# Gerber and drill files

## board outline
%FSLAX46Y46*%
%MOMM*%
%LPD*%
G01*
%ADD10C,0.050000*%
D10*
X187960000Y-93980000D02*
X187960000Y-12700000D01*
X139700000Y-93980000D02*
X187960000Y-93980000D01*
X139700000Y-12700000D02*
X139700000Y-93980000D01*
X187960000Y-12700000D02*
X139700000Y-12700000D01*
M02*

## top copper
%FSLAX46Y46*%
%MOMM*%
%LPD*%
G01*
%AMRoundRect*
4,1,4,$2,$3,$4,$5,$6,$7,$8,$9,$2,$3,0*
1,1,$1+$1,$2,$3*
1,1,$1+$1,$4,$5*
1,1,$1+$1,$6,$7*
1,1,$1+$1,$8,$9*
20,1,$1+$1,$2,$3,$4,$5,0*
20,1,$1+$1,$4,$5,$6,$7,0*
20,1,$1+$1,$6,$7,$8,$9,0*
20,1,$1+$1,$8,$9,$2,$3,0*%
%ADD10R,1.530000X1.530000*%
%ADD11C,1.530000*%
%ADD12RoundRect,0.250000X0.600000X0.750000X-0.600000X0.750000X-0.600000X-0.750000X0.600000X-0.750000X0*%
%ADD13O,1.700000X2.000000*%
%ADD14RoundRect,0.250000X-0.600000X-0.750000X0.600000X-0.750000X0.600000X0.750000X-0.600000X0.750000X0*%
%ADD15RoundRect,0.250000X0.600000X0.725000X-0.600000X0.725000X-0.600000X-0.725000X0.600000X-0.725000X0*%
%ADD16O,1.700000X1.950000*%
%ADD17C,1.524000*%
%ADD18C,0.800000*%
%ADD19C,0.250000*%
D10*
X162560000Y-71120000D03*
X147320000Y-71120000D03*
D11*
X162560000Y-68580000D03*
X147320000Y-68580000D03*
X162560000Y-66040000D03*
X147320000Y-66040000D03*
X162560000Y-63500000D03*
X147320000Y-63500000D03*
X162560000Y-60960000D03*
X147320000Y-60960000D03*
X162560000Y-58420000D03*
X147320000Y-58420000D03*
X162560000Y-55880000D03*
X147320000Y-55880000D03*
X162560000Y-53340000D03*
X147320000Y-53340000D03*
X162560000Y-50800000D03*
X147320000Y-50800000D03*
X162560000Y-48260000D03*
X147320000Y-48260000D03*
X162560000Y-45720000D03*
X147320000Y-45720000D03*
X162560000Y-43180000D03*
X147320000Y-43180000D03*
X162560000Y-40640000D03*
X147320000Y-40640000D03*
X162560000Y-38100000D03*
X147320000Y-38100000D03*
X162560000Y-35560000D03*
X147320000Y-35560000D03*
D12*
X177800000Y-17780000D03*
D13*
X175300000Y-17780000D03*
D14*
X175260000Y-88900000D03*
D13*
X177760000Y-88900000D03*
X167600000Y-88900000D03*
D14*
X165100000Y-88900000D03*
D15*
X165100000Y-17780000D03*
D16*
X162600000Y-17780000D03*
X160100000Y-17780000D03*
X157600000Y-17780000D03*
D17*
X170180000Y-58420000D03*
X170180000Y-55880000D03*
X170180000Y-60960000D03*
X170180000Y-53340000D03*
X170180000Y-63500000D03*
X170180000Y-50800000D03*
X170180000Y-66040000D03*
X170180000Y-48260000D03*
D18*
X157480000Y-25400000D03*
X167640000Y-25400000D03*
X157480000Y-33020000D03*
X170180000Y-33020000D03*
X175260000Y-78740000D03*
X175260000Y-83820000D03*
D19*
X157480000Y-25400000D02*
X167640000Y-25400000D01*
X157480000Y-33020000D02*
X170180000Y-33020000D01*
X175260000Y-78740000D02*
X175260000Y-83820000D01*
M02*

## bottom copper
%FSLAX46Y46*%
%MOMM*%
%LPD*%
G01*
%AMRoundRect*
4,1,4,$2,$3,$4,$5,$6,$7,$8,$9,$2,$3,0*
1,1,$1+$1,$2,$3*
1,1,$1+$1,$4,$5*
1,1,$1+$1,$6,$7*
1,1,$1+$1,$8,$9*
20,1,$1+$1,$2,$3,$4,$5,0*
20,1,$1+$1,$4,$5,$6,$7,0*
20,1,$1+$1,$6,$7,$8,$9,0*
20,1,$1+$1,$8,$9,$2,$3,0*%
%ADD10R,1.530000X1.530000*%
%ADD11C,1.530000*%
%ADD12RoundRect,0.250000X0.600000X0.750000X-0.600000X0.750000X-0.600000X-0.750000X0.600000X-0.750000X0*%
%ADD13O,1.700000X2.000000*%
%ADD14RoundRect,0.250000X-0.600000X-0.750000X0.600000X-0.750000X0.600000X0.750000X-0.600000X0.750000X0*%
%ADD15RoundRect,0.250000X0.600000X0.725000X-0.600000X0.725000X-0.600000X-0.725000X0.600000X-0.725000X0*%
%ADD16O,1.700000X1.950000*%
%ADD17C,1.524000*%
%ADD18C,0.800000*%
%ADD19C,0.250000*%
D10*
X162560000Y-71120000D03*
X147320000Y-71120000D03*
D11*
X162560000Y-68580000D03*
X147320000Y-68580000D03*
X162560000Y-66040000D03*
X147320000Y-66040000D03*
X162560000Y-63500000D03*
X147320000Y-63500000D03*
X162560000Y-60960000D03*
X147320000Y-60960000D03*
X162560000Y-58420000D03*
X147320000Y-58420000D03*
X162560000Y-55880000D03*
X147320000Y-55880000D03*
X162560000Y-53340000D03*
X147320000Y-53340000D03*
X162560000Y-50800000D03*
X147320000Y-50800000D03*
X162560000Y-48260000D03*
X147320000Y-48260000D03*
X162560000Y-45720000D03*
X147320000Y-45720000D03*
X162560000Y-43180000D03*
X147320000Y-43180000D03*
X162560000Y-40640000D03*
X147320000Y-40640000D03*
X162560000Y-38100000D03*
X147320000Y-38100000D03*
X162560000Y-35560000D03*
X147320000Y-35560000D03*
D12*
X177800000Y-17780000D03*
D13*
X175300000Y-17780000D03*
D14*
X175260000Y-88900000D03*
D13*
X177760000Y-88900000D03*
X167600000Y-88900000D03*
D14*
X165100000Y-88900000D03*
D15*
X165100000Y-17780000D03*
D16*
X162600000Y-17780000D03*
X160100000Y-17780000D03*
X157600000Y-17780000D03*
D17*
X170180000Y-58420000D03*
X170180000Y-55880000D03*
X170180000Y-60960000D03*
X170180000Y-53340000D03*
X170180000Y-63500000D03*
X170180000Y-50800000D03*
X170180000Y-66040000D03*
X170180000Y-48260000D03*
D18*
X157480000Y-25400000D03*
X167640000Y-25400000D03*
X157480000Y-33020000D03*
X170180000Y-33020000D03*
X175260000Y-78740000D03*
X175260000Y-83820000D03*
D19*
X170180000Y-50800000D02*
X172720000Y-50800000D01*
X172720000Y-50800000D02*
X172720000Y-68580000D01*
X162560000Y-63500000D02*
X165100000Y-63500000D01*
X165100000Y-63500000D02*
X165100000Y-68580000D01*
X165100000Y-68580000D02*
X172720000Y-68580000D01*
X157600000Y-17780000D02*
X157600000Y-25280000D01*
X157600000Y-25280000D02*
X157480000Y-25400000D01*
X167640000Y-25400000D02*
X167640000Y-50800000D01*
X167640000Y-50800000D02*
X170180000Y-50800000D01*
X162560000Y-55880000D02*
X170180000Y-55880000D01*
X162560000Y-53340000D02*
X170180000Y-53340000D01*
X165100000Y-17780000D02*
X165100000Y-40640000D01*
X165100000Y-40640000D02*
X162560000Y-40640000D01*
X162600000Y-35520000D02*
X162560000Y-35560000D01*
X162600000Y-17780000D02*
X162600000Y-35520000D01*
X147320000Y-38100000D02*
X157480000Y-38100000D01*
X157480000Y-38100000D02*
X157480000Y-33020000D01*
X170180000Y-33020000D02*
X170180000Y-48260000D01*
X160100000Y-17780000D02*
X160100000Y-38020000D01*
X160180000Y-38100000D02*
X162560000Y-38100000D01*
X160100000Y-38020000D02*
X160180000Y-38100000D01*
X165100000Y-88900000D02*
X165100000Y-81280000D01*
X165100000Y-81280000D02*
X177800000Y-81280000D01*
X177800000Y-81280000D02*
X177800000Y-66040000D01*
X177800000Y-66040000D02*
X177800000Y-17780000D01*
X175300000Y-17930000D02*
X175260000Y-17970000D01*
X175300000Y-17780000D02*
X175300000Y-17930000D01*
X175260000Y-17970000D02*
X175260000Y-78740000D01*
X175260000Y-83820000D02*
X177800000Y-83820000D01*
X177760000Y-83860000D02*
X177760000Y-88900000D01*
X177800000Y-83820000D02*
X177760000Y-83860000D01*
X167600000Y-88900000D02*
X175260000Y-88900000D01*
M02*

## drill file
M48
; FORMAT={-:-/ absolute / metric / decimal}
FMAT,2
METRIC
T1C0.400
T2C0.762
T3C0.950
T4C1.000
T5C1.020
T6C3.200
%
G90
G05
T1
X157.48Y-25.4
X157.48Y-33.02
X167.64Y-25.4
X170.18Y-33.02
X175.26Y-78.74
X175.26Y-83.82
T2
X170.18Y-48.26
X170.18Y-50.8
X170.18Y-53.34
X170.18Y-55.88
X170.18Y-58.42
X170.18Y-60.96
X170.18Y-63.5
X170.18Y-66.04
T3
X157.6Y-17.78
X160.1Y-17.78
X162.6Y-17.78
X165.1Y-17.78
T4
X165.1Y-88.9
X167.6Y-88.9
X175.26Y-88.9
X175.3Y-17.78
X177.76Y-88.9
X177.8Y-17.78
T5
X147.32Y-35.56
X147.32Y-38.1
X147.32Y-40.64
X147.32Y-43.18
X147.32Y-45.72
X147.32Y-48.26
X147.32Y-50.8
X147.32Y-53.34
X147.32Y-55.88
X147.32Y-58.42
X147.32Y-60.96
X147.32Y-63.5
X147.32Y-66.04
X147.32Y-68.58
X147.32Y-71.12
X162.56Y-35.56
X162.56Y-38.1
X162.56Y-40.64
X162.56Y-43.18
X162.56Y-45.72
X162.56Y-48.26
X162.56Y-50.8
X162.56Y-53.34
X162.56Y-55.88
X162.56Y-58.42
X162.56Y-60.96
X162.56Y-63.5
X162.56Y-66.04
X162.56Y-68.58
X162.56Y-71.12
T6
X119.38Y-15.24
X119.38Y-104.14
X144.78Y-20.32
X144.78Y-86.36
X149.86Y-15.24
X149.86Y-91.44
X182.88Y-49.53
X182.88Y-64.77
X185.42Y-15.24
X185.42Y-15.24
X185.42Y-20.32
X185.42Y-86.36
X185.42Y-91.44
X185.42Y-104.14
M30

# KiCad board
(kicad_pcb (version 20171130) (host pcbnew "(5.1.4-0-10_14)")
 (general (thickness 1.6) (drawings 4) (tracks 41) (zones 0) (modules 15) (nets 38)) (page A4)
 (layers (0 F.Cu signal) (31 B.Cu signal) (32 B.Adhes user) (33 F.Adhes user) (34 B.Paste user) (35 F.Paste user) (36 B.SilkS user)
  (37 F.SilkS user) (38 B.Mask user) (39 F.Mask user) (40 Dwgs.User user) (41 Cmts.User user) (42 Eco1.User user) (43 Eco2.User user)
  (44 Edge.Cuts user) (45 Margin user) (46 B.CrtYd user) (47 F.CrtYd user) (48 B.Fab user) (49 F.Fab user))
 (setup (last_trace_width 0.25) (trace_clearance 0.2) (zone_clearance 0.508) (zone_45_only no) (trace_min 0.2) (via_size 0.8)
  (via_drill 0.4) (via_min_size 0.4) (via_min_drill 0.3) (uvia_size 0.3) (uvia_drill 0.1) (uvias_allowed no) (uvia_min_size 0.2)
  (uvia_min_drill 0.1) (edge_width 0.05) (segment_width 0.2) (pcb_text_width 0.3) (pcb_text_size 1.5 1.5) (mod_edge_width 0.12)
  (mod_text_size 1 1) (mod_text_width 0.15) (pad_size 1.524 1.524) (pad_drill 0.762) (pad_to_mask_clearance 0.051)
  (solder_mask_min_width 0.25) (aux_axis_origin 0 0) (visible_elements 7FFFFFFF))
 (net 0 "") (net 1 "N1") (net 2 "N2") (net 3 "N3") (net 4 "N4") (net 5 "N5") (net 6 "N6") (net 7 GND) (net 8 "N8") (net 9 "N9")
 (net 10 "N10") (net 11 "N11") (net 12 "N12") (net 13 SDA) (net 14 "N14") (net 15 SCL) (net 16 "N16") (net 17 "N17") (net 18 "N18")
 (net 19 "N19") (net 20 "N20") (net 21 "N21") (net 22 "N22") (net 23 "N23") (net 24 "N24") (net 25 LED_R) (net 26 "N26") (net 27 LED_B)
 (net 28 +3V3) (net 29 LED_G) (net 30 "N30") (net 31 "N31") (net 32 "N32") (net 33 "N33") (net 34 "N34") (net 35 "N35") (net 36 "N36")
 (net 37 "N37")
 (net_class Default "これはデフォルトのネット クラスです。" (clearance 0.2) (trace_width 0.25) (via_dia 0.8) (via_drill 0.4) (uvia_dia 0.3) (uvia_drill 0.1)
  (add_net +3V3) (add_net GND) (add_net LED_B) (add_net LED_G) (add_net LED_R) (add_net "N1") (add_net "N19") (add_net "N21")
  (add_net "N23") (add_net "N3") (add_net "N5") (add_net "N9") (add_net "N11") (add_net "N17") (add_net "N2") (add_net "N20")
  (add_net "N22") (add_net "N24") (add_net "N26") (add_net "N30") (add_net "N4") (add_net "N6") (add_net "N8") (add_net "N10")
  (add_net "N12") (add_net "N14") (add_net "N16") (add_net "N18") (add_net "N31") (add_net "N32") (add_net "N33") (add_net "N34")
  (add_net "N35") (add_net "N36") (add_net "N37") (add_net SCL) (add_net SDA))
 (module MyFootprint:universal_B (layer F.Cu) (at 152.4 58.42 90)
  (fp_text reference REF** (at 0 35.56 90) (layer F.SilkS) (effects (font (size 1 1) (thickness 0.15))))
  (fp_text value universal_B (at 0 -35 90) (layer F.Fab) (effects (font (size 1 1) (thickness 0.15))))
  (pad "" np_thru_hole circle (at 43.18 -33.02 90) (size 3.2 3.2) (drill 3.2) (layers *.Cu *.Mask))
  (pad "" np_thru_hole circle (at 43.18 33.02 90) (size 3.2 3.2) (drill 3.2) (layers *.Cu *.Mask))
  (pad "" np_thru_hole circle (at -45.72 33.02 90) (size 3.2 3.2) (drill 3.2) (layers *.Cu *.Mask))
  (pad "" np_thru_hole circle (at -45.72 -33.02 90) (size 3.2 3.2) (drill 3.2) (layers *.Cu *.Mask)))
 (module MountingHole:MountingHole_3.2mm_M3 (layer F.Cu) (at 144.78 86.36)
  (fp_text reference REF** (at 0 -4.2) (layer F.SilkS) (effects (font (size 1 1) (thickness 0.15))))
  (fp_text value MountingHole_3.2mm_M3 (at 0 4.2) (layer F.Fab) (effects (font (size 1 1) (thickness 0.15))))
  (pad 1 np_thru_hole circle (at 0 0) (size 3.2 3.2) (drill 3.2) (layers *.Cu *.Mask)))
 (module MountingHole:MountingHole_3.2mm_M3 (layer F.Cu) (at 185.42 86.36)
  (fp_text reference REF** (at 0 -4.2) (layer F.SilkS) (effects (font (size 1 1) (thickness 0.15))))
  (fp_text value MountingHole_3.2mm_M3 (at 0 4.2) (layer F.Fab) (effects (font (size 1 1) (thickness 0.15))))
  (pad 1 np_thru_hole circle (at 0 0) (size 3.2 3.2) (drill 3.2) (layers *.Cu *.Mask)))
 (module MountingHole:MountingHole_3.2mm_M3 (layer F.Cu) (at 144.78 20.32)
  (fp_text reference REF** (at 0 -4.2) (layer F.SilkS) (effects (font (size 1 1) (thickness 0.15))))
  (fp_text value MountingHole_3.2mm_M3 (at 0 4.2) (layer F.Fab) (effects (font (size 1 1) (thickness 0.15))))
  (pad 1 np_thru_hole circle (at 0 0) (size 3.2 3.2) (drill 3.2) (layers *.Cu *.Mask)))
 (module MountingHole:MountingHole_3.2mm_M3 (layer F.Cu) (at 185.42 20.32)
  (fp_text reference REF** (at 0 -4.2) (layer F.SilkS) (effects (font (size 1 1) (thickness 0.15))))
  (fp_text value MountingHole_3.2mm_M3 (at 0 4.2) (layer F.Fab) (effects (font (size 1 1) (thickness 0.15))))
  (pad 1 np_thru_hole circle (at 0 0) (size 3.2 3.2) (drill 3.2) (layers *.Cu *.Mask)))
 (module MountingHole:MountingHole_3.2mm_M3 (layer F.Cu) (at 149.86 91.44)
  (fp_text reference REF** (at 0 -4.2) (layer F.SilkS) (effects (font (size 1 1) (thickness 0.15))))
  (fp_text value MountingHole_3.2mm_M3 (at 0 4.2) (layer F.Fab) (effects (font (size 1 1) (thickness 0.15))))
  (pad 1 np_thru_hole circle (at 0 0) (size 3.2 3.2) (drill 3.2) (layers *.Cu *.Mask)))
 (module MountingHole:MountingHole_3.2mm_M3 (layer F.Cu) (at 185.42 91.44)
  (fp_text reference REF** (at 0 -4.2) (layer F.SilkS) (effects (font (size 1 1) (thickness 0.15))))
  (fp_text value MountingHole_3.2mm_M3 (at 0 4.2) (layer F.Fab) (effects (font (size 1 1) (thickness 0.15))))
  (pad 1 np_thru_hole circle (at 0 0) (size 3.2 3.2) (drill 3.2) (layers *.Cu *.Mask)))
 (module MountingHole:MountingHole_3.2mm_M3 (layer F.Cu) (at 149.86 15.24)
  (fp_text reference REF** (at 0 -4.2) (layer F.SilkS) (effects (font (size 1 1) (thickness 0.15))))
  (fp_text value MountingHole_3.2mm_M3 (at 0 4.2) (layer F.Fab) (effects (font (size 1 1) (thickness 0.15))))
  (pad 1 np_thru_hole circle (at 0 0) (size 3.2 3.2) (drill 3.2) (layers *.Cu *.Mask)))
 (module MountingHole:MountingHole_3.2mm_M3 (layer F.Cu) (at 185.42 15.24)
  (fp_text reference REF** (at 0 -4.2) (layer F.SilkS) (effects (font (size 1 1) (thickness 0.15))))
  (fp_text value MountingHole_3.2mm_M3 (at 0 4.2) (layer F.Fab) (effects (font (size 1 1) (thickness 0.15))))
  (pad 1 np_thru_hole circle (at 0 0) (size 3.2 3.2) (drill 3.2) (layers *.Cu *.Mask)))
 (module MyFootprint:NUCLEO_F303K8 (layer F.Cu) (at 154.94 53.34 180)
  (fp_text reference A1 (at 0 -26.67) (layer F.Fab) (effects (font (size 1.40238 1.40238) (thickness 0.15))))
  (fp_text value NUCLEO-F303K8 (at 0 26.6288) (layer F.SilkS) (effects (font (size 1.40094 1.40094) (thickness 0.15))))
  (pad 3.1 thru_hole rect (at -7.62 -17.78 180) (size 1.53 1.53) (drill 1.02) (layers *.Cu *.Mask) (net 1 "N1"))
  (pad 4.1 thru_hole rect (at 7.62 -17.78 180) (size 1.53 1.53) (drill 1.02) (layers *.Cu *.Mask) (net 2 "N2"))
  (pad 3.2 thru_hole circle (at -7.62 -15.24 180) (size 1.53 1.53) (drill 1.02) (layers *.Cu *.Mask) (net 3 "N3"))
  (pad 4.2 thru_hole circle (at 7.62 -15.24 180) (size 1.53 1.53) (drill 1.02) (layers *.Cu *.Mask) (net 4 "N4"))
  (pad 3.3 thru_hole circle (at -7.62 -12.7 180) (size 1.53 1.53) (drill 1.02) (layers *.Cu *.Mask) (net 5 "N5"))
  (pad 4.3 thru_hole circle (at 7.62 -12.7 180) (size 1.53 1.53) (drill 1.02) (layers *.Cu *.Mask) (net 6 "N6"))
  (pad 3.4 thru_hole circle (at -7.62 -10.16 180) (size 1.53 1.53) (drill 1.02) (layers *.Cu *.Mask) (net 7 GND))
  (pad 4.4 thru_hole circle (at 7.62 -10.16 180) (size 1.53 1.53) (drill 1.02) (layers *.Cu *.Mask) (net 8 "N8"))
  (pad 3.5 thru_hole circle (at -7.62 -7.62 180) (size 1.53 1.53) (drill 1.02) (layers *.Cu *.Mask) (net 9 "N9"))
  (pad 4.5 thru_hole circle (at 7.62 -7.62 180) (size 1.53 1.53) (drill 1.02) (layers *.Cu *.Mask) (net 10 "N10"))
  (pad 3.6 thru_hole circle (at -7.62 -5.08 180) (size 1.53 1.53) (drill 1.02) (layers *.Cu *.Mask) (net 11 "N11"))
  (pad 4.6 thru_hole circle (at 7.62 -5.08 180) (size 1.53 1.53) (drill 1.02) (layers *.Cu *.Mask) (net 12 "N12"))
  (pad 3.7 thru_hole circle (at -7.62 -2.54 180) (size 1.53 1.53) (drill 1.02) (layers *.Cu *.Mask) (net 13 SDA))
  (pad 4.7 thru_hole circle (at 7.62 -2.54 180) (size 1.53 1.53) (drill 1.02) (layers *.Cu *.Mask) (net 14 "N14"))
  (pad 3.8 thru_hole circle (at -7.62 0 180) (size 1.53 1.53) (drill 1.02) (layers *.Cu *.Mask) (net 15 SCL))
  (pad 4.8 thru_hole circle (at 7.62 0 180) (size 1.53 1.53) (drill 1.02) (layers *.Cu *.Mask) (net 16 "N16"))
  (pad 3.9 thru_hole circle (at -7.62 2.54 180) (size 1.53 1.53) (drill 1.02) (layers *.Cu *.Mask) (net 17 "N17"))
  (pad 4.9 thru_hole circle (at 7.62 2.54 180) (size 1.53 1.53) (drill 1.02) (layers *.Cu *.Mask) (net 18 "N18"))
  (pad 3.10 thru_hole circle (at -7.62 5.08 180) (size 1.53 1.53) (drill 1.02) (layers *.Cu *.Mask) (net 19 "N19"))
  (pad 4.10 thru_hole circle (at 7.62 5.08 180) (size 1.53 1.53) (drill 1.02) (layers *.Cu *.Mask) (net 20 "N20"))
  (pad 3.11 thru_hole circle (at -7.62 7.62 180) (size 1.53 1.53) (drill 1.02) (layers *.Cu *.Mask) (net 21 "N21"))
  (pad 4.11 thru_hole circle (at 7.62 7.62 180) (size 1.53 1.53) (drill 1.02) (layers *.Cu *.Mask) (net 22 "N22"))
  (pad 3.12 thru_hole circle (at -7.62 10.16 180) (size 1.53 1.53) (drill 1.02) (layers *.Cu *.Mask) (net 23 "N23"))
  (pad 4.12 thru_hole circle (at 7.62 10.16 180) (size 1.53 1.53) (drill 1.02) (layers *.Cu *.Mask) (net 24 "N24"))
  (pad 3.13 thru_hole circle (at -7.62 12.7 180) (size 1.53 1.53) (drill 1.02) (layers *.Cu *.Mask) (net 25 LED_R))
  (pad 4.13 thru_hole circle (at 7.62 12.7 180) (size 1.53 1.53) (drill 1.02) (layers *.Cu *.Mask) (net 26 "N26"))
  (pad 3.14 thru_hole circle (at -7.62 15.24 180) (size 1.53 1.53) (drill 1.02) (layers *.Cu *.Mask) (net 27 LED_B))
  (pad 4.14 thru_hole circle (at 7.62 15.24 180) (size 1.53 1.53) (drill 1.02) (layers *.Cu *.Mask) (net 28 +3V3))
  (pad 3.15 thru_hole circle (at -7.62 17.78 180) (size 1.53 1.53) (drill 1.02) (layers *.Cu *.Mask) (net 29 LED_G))
  (pad 4.15 thru_hole circle (at 7.62 17.78 180) (size 1.53 1.53) (drill 1.02) (layers *.Cu *.Mask) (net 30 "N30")))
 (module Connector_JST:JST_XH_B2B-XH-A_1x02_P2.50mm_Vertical (layer F.Cu) (at 177.8 17.78 180)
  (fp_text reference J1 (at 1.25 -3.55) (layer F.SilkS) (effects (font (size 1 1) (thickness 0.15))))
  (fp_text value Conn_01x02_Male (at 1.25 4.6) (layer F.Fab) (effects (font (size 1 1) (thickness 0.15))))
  (pad 1 thru_hole roundrect (at 0 0 180) (size 1.7 2) (drill 1) (layers *.Cu *.Mask) (roundrect_rratio 0.147059) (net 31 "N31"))
  (pad 2 thru_hole oval (at 2.5 0 180) (size 1.7 2) (drill 1) (layers *.Cu *.Mask) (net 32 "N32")))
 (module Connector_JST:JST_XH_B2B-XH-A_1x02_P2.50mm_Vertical (layer F.Cu) (at 175.26 88.9)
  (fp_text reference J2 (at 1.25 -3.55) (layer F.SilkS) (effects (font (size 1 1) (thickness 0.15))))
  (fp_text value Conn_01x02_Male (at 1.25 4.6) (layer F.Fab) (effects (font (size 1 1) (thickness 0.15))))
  (pad 1 thru_hole roundrect (at 0 0) (size 1.7 2) (drill 1) (layers *.Cu *.Mask) (roundrect_rratio 0.147059) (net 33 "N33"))
  (pad 2 thru_hole oval (at 2.5 0) (size 1.7 2) (drill 1) (layers *.Cu *.Mask) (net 32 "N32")))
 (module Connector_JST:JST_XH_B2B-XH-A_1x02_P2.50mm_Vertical (layer F.Cu) (at 165.1 88.9)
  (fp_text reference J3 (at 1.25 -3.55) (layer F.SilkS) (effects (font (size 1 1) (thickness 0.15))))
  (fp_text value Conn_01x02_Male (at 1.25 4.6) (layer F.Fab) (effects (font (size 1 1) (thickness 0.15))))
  (pad 2 thru_hole oval (at 2.5 0) (size 1.7 2) (drill 1) (layers *.Cu *.Mask) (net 33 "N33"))
  (pad 1 thru_hole roundrect (at 0 0) (size 1.7 2) (drill 1) (layers *.Cu *.Mask) (roundrect_rratio 0.147059) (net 31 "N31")))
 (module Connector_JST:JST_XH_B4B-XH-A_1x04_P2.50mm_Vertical (layer F.Cu) (at 165.1 17.78 180)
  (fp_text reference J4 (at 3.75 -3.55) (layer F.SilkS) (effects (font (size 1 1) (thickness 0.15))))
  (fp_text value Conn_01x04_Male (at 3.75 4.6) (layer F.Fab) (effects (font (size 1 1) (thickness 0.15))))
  (pad 1 thru_hole roundrect (at 0 0 180) (size 1.7 1.95) (drill 0.95) (layers *.Cu *.Mask) (roundrect_rratio 0.147059) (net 25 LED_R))
  (pad 2 thru_hole oval (at 2.5 0 180) (size 1.7 1.95) (drill 0.95) (layers *.Cu *.Mask) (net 29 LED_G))
  (pad 3 thru_hole oval (at 5 0 180) (size 1.7 1.95) (drill 0.95) (layers *.Cu *.Mask) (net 27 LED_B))
  (pad 4 thru_hole oval (at 7.5 0 180) (size 1.7 1.95) (drill 0.95) (layers *.Cu *.Mask) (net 7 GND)))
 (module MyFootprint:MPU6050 (layer F.Cu) (at 175.26 58.42)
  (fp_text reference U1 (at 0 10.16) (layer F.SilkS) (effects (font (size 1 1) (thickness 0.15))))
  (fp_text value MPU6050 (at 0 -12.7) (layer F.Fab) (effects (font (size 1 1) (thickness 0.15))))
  (pad 5 thru_hole circle (at -5.08 0) (size 1.524 1.524) (drill 0.762) (layers *.Cu *.Mask) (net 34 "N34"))
  (pad 4 thru_hole circle (at -5.08 -2.54) (size 1.524 1.524) (drill 0.762) (layers *.Cu *.Mask) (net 13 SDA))
  (pad 6 thru_hole circle (at -5.08 2.54) (size 1.524 1.524) (drill 0.762) (layers *.Cu *.Mask) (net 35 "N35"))
  (pad 3 thru_hole circle (at -5.08 -5.08) (size 1.524 1.524) (drill 0.762) (layers *.Cu *.Mask) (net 15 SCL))
  (pad 7 thru_hole circle (at -5.08 5.08) (size 1.524 1.524) (drill 0.762) (layers *.Cu *.Mask) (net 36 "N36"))
  (pad 2 thru_hole circle (at -5.08 -7.62) (size 1.524 1.524) (drill 0.762) (layers *.Cu *.Mask) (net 7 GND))
  (pad 8 thru_hole circle (at -5.08 7.62) (size 1.524 1.524) (drill 0.762) (layers *.Cu *.Mask) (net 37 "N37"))
  (pad 1 thru_hole circle (at -5.08 -10.16) (size 1.524 1.524) (drill 0.762) (layers *.Cu *.Mask) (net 28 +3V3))
  (pad "" np_thru_hole circle (at 7.62 -8.89) (size 3.2 3.2) (drill 3.2) (layers *.Cu *.Mask))
  (pad "" np_thru_hole circle (at 7.62 6.35) (size 3.2 3.2) (drill 3.2) (layers *.Cu *.Mask)))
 (gr_line (start 187.96 93.98) (end 187.96 12.7) (layer Edge.Cuts) (width 0.05))
 (gr_line (start 139.7 93.98) (end 187.96 93.98) (layer Edge.Cuts) (width 0.05))
 (gr_line (start 139.7 12.7) (end 139.7 93.98) (layer Edge.Cuts) (width 0.05))
 (gr_line (start 187.96 12.7) (end 139.7 12.7) (layer Edge.Cuts) (width 0.05))
 (segment (start 170.18 50.8) (end 172.72 50.8) (width 0.25) (layer B.Cu) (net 7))
 (segment (start 172.72 50.8) (end 172.72 68.58) (width 0.25) (layer B.Cu) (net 7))
 (segment (start 162.56 63.5) (end 165.1 63.5) (width 0.25) (layer B.Cu) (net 7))
 (segment (start 165.1 63.5) (end 165.1 68.58) (width 0.25) (layer B.Cu) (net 7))
 (segment (start 165.1 68.58) (end 172.72 68.58) (width 0.25) (layer B.Cu) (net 7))
 (via (at 157.48 25.4) (size 0.8) (drill 0.4) (layers F.Cu B.Cu) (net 7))
 (segment (start 157.6 17.78) (end 157.6 25.28) (width 0.25) (layer B.Cu) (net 7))
 (segment (start 157.6 25.28) (end 157.48 25.4) (width 0.25) (layer B.Cu) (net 7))
 (via (at 167.64 25.4) (size 0.8) (drill 0.4) (layers F.Cu B.Cu) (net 7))
 (segment (start 157.48 25.4) (end 167.64 25.4) (width 0.25) (layer F.Cu) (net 7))
 (segment (start 167.64 25.4) (end 167.64 50.8) (width 0.25) (layer B.Cu) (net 7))
 (segment (start 167.64 50.8) (end 170.18 50.8) (width 0.25) (layer B.Cu) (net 7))
 (segment (start 162.56 55.88) (end 170.18 55.88) (width 0.25) (layer B.Cu) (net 13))
 (segment (start 162.56 53.34) (end 170.18 53.34) (width 0.25) (layer B.Cu) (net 15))
 (segment (start 165.1 17.78) (end 165.1 40.64) (width 0.25) (layer B.Cu) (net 25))
 (segment (start 165.1 40.64) (end 162.56 40.64) (width 0.25) (layer B.Cu) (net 25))
 (segment (start 162.6 35.52) (end 162.56 35.56) (width 0.25) (layer B.Cu) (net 29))
 (segment (start 162.6 17.78) (end 162.6 35.52) (width 0.25) (layer B.Cu) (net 29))
 (segment (start 147.32 38.1) (end 157.48 38.1) (width 0.25) (layer B.Cu) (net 28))
 (via (at 157.48 33.02) (size 0.8) (drill 0.4) (layers F.Cu B.Cu) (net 28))
 (segment (start 157.48 38.1) (end 157.48 33.02) (width 0.25) (layer B.Cu) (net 28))
 (via (at 170.18 33.02) (size 0.8) (drill 0.4) (layers F.Cu B.Cu) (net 28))
 (segment (start 157.48 33.02) (end 170.18 33.02) (width 0.25) (layer F.Cu) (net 28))
 (segment (start 170.18 33.02) (end 170.18 48.26) (width 0.25) (layer B.Cu) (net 28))
 (segment (start 160.1 17.78) (end 160.1 38.02) (width 0.25) (layer B.Cu) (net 27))
 (segment (start 160.18 38.1) (end 162.56 38.1) (width 0.25) (layer B.Cu) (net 27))
 (segment (start 160.1 38.02) (end 160.18 38.1) (width 0.25) (layer B.Cu) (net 27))
 (segment (start 165.1 88.9) (end 165.1 81.28) (width 0.25) (layer B.Cu) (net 31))
 (segment (start 165.1 81.28) (end 177.8 81.28) (width 0.25) (layer B.Cu) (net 31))
 (segment (start 177.8 81.28) (end 177.8 66.04) (width 0.25) (layer B.Cu) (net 31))
 (segment (start 177.8 66.04) (end 177.8 17.78) (width 0.25) (layer B.Cu) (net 31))
 (segment (start 175.3 17.93) (end 175.26 17.97) (width 0.25) (layer B.Cu) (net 32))
 (segment (start 175.3 17.78) (end 175.3 17.93) (width 0.25) (layer B.Cu) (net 32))
 (via (at 175.26 78.74) (size 0.8) (drill 0.4) (layers F.Cu B.Cu) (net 32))
 (segment (start 175.26 17.97) (end 175.26 78.74) (width 0.25) (layer B.Cu) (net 32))
 (via (at 175.26 83.82) (size 0.8) (drill 0.4) (layers F.Cu B.Cu) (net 32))
 (segment (start 175.26 78.74) (end 175.26 83.82) (width 0.25) (layer F.Cu) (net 32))
 (segment (start 175.26 83.82) (end 177.8 83.82) (width 0.25) (layer B.Cu) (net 32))
 (segment (start 177.76 83.86) (end 177.76 88.9) (width 0.25) (layer B.Cu) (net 32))
 (segment (start 177.8 83.82) (end 177.76 83.86) (width 0.25) (layer B.Cu) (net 32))
 (segment (start 167.6 88.9) (end 175.26 88.9) (width 0.25) (layer B.Cu) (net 33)))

